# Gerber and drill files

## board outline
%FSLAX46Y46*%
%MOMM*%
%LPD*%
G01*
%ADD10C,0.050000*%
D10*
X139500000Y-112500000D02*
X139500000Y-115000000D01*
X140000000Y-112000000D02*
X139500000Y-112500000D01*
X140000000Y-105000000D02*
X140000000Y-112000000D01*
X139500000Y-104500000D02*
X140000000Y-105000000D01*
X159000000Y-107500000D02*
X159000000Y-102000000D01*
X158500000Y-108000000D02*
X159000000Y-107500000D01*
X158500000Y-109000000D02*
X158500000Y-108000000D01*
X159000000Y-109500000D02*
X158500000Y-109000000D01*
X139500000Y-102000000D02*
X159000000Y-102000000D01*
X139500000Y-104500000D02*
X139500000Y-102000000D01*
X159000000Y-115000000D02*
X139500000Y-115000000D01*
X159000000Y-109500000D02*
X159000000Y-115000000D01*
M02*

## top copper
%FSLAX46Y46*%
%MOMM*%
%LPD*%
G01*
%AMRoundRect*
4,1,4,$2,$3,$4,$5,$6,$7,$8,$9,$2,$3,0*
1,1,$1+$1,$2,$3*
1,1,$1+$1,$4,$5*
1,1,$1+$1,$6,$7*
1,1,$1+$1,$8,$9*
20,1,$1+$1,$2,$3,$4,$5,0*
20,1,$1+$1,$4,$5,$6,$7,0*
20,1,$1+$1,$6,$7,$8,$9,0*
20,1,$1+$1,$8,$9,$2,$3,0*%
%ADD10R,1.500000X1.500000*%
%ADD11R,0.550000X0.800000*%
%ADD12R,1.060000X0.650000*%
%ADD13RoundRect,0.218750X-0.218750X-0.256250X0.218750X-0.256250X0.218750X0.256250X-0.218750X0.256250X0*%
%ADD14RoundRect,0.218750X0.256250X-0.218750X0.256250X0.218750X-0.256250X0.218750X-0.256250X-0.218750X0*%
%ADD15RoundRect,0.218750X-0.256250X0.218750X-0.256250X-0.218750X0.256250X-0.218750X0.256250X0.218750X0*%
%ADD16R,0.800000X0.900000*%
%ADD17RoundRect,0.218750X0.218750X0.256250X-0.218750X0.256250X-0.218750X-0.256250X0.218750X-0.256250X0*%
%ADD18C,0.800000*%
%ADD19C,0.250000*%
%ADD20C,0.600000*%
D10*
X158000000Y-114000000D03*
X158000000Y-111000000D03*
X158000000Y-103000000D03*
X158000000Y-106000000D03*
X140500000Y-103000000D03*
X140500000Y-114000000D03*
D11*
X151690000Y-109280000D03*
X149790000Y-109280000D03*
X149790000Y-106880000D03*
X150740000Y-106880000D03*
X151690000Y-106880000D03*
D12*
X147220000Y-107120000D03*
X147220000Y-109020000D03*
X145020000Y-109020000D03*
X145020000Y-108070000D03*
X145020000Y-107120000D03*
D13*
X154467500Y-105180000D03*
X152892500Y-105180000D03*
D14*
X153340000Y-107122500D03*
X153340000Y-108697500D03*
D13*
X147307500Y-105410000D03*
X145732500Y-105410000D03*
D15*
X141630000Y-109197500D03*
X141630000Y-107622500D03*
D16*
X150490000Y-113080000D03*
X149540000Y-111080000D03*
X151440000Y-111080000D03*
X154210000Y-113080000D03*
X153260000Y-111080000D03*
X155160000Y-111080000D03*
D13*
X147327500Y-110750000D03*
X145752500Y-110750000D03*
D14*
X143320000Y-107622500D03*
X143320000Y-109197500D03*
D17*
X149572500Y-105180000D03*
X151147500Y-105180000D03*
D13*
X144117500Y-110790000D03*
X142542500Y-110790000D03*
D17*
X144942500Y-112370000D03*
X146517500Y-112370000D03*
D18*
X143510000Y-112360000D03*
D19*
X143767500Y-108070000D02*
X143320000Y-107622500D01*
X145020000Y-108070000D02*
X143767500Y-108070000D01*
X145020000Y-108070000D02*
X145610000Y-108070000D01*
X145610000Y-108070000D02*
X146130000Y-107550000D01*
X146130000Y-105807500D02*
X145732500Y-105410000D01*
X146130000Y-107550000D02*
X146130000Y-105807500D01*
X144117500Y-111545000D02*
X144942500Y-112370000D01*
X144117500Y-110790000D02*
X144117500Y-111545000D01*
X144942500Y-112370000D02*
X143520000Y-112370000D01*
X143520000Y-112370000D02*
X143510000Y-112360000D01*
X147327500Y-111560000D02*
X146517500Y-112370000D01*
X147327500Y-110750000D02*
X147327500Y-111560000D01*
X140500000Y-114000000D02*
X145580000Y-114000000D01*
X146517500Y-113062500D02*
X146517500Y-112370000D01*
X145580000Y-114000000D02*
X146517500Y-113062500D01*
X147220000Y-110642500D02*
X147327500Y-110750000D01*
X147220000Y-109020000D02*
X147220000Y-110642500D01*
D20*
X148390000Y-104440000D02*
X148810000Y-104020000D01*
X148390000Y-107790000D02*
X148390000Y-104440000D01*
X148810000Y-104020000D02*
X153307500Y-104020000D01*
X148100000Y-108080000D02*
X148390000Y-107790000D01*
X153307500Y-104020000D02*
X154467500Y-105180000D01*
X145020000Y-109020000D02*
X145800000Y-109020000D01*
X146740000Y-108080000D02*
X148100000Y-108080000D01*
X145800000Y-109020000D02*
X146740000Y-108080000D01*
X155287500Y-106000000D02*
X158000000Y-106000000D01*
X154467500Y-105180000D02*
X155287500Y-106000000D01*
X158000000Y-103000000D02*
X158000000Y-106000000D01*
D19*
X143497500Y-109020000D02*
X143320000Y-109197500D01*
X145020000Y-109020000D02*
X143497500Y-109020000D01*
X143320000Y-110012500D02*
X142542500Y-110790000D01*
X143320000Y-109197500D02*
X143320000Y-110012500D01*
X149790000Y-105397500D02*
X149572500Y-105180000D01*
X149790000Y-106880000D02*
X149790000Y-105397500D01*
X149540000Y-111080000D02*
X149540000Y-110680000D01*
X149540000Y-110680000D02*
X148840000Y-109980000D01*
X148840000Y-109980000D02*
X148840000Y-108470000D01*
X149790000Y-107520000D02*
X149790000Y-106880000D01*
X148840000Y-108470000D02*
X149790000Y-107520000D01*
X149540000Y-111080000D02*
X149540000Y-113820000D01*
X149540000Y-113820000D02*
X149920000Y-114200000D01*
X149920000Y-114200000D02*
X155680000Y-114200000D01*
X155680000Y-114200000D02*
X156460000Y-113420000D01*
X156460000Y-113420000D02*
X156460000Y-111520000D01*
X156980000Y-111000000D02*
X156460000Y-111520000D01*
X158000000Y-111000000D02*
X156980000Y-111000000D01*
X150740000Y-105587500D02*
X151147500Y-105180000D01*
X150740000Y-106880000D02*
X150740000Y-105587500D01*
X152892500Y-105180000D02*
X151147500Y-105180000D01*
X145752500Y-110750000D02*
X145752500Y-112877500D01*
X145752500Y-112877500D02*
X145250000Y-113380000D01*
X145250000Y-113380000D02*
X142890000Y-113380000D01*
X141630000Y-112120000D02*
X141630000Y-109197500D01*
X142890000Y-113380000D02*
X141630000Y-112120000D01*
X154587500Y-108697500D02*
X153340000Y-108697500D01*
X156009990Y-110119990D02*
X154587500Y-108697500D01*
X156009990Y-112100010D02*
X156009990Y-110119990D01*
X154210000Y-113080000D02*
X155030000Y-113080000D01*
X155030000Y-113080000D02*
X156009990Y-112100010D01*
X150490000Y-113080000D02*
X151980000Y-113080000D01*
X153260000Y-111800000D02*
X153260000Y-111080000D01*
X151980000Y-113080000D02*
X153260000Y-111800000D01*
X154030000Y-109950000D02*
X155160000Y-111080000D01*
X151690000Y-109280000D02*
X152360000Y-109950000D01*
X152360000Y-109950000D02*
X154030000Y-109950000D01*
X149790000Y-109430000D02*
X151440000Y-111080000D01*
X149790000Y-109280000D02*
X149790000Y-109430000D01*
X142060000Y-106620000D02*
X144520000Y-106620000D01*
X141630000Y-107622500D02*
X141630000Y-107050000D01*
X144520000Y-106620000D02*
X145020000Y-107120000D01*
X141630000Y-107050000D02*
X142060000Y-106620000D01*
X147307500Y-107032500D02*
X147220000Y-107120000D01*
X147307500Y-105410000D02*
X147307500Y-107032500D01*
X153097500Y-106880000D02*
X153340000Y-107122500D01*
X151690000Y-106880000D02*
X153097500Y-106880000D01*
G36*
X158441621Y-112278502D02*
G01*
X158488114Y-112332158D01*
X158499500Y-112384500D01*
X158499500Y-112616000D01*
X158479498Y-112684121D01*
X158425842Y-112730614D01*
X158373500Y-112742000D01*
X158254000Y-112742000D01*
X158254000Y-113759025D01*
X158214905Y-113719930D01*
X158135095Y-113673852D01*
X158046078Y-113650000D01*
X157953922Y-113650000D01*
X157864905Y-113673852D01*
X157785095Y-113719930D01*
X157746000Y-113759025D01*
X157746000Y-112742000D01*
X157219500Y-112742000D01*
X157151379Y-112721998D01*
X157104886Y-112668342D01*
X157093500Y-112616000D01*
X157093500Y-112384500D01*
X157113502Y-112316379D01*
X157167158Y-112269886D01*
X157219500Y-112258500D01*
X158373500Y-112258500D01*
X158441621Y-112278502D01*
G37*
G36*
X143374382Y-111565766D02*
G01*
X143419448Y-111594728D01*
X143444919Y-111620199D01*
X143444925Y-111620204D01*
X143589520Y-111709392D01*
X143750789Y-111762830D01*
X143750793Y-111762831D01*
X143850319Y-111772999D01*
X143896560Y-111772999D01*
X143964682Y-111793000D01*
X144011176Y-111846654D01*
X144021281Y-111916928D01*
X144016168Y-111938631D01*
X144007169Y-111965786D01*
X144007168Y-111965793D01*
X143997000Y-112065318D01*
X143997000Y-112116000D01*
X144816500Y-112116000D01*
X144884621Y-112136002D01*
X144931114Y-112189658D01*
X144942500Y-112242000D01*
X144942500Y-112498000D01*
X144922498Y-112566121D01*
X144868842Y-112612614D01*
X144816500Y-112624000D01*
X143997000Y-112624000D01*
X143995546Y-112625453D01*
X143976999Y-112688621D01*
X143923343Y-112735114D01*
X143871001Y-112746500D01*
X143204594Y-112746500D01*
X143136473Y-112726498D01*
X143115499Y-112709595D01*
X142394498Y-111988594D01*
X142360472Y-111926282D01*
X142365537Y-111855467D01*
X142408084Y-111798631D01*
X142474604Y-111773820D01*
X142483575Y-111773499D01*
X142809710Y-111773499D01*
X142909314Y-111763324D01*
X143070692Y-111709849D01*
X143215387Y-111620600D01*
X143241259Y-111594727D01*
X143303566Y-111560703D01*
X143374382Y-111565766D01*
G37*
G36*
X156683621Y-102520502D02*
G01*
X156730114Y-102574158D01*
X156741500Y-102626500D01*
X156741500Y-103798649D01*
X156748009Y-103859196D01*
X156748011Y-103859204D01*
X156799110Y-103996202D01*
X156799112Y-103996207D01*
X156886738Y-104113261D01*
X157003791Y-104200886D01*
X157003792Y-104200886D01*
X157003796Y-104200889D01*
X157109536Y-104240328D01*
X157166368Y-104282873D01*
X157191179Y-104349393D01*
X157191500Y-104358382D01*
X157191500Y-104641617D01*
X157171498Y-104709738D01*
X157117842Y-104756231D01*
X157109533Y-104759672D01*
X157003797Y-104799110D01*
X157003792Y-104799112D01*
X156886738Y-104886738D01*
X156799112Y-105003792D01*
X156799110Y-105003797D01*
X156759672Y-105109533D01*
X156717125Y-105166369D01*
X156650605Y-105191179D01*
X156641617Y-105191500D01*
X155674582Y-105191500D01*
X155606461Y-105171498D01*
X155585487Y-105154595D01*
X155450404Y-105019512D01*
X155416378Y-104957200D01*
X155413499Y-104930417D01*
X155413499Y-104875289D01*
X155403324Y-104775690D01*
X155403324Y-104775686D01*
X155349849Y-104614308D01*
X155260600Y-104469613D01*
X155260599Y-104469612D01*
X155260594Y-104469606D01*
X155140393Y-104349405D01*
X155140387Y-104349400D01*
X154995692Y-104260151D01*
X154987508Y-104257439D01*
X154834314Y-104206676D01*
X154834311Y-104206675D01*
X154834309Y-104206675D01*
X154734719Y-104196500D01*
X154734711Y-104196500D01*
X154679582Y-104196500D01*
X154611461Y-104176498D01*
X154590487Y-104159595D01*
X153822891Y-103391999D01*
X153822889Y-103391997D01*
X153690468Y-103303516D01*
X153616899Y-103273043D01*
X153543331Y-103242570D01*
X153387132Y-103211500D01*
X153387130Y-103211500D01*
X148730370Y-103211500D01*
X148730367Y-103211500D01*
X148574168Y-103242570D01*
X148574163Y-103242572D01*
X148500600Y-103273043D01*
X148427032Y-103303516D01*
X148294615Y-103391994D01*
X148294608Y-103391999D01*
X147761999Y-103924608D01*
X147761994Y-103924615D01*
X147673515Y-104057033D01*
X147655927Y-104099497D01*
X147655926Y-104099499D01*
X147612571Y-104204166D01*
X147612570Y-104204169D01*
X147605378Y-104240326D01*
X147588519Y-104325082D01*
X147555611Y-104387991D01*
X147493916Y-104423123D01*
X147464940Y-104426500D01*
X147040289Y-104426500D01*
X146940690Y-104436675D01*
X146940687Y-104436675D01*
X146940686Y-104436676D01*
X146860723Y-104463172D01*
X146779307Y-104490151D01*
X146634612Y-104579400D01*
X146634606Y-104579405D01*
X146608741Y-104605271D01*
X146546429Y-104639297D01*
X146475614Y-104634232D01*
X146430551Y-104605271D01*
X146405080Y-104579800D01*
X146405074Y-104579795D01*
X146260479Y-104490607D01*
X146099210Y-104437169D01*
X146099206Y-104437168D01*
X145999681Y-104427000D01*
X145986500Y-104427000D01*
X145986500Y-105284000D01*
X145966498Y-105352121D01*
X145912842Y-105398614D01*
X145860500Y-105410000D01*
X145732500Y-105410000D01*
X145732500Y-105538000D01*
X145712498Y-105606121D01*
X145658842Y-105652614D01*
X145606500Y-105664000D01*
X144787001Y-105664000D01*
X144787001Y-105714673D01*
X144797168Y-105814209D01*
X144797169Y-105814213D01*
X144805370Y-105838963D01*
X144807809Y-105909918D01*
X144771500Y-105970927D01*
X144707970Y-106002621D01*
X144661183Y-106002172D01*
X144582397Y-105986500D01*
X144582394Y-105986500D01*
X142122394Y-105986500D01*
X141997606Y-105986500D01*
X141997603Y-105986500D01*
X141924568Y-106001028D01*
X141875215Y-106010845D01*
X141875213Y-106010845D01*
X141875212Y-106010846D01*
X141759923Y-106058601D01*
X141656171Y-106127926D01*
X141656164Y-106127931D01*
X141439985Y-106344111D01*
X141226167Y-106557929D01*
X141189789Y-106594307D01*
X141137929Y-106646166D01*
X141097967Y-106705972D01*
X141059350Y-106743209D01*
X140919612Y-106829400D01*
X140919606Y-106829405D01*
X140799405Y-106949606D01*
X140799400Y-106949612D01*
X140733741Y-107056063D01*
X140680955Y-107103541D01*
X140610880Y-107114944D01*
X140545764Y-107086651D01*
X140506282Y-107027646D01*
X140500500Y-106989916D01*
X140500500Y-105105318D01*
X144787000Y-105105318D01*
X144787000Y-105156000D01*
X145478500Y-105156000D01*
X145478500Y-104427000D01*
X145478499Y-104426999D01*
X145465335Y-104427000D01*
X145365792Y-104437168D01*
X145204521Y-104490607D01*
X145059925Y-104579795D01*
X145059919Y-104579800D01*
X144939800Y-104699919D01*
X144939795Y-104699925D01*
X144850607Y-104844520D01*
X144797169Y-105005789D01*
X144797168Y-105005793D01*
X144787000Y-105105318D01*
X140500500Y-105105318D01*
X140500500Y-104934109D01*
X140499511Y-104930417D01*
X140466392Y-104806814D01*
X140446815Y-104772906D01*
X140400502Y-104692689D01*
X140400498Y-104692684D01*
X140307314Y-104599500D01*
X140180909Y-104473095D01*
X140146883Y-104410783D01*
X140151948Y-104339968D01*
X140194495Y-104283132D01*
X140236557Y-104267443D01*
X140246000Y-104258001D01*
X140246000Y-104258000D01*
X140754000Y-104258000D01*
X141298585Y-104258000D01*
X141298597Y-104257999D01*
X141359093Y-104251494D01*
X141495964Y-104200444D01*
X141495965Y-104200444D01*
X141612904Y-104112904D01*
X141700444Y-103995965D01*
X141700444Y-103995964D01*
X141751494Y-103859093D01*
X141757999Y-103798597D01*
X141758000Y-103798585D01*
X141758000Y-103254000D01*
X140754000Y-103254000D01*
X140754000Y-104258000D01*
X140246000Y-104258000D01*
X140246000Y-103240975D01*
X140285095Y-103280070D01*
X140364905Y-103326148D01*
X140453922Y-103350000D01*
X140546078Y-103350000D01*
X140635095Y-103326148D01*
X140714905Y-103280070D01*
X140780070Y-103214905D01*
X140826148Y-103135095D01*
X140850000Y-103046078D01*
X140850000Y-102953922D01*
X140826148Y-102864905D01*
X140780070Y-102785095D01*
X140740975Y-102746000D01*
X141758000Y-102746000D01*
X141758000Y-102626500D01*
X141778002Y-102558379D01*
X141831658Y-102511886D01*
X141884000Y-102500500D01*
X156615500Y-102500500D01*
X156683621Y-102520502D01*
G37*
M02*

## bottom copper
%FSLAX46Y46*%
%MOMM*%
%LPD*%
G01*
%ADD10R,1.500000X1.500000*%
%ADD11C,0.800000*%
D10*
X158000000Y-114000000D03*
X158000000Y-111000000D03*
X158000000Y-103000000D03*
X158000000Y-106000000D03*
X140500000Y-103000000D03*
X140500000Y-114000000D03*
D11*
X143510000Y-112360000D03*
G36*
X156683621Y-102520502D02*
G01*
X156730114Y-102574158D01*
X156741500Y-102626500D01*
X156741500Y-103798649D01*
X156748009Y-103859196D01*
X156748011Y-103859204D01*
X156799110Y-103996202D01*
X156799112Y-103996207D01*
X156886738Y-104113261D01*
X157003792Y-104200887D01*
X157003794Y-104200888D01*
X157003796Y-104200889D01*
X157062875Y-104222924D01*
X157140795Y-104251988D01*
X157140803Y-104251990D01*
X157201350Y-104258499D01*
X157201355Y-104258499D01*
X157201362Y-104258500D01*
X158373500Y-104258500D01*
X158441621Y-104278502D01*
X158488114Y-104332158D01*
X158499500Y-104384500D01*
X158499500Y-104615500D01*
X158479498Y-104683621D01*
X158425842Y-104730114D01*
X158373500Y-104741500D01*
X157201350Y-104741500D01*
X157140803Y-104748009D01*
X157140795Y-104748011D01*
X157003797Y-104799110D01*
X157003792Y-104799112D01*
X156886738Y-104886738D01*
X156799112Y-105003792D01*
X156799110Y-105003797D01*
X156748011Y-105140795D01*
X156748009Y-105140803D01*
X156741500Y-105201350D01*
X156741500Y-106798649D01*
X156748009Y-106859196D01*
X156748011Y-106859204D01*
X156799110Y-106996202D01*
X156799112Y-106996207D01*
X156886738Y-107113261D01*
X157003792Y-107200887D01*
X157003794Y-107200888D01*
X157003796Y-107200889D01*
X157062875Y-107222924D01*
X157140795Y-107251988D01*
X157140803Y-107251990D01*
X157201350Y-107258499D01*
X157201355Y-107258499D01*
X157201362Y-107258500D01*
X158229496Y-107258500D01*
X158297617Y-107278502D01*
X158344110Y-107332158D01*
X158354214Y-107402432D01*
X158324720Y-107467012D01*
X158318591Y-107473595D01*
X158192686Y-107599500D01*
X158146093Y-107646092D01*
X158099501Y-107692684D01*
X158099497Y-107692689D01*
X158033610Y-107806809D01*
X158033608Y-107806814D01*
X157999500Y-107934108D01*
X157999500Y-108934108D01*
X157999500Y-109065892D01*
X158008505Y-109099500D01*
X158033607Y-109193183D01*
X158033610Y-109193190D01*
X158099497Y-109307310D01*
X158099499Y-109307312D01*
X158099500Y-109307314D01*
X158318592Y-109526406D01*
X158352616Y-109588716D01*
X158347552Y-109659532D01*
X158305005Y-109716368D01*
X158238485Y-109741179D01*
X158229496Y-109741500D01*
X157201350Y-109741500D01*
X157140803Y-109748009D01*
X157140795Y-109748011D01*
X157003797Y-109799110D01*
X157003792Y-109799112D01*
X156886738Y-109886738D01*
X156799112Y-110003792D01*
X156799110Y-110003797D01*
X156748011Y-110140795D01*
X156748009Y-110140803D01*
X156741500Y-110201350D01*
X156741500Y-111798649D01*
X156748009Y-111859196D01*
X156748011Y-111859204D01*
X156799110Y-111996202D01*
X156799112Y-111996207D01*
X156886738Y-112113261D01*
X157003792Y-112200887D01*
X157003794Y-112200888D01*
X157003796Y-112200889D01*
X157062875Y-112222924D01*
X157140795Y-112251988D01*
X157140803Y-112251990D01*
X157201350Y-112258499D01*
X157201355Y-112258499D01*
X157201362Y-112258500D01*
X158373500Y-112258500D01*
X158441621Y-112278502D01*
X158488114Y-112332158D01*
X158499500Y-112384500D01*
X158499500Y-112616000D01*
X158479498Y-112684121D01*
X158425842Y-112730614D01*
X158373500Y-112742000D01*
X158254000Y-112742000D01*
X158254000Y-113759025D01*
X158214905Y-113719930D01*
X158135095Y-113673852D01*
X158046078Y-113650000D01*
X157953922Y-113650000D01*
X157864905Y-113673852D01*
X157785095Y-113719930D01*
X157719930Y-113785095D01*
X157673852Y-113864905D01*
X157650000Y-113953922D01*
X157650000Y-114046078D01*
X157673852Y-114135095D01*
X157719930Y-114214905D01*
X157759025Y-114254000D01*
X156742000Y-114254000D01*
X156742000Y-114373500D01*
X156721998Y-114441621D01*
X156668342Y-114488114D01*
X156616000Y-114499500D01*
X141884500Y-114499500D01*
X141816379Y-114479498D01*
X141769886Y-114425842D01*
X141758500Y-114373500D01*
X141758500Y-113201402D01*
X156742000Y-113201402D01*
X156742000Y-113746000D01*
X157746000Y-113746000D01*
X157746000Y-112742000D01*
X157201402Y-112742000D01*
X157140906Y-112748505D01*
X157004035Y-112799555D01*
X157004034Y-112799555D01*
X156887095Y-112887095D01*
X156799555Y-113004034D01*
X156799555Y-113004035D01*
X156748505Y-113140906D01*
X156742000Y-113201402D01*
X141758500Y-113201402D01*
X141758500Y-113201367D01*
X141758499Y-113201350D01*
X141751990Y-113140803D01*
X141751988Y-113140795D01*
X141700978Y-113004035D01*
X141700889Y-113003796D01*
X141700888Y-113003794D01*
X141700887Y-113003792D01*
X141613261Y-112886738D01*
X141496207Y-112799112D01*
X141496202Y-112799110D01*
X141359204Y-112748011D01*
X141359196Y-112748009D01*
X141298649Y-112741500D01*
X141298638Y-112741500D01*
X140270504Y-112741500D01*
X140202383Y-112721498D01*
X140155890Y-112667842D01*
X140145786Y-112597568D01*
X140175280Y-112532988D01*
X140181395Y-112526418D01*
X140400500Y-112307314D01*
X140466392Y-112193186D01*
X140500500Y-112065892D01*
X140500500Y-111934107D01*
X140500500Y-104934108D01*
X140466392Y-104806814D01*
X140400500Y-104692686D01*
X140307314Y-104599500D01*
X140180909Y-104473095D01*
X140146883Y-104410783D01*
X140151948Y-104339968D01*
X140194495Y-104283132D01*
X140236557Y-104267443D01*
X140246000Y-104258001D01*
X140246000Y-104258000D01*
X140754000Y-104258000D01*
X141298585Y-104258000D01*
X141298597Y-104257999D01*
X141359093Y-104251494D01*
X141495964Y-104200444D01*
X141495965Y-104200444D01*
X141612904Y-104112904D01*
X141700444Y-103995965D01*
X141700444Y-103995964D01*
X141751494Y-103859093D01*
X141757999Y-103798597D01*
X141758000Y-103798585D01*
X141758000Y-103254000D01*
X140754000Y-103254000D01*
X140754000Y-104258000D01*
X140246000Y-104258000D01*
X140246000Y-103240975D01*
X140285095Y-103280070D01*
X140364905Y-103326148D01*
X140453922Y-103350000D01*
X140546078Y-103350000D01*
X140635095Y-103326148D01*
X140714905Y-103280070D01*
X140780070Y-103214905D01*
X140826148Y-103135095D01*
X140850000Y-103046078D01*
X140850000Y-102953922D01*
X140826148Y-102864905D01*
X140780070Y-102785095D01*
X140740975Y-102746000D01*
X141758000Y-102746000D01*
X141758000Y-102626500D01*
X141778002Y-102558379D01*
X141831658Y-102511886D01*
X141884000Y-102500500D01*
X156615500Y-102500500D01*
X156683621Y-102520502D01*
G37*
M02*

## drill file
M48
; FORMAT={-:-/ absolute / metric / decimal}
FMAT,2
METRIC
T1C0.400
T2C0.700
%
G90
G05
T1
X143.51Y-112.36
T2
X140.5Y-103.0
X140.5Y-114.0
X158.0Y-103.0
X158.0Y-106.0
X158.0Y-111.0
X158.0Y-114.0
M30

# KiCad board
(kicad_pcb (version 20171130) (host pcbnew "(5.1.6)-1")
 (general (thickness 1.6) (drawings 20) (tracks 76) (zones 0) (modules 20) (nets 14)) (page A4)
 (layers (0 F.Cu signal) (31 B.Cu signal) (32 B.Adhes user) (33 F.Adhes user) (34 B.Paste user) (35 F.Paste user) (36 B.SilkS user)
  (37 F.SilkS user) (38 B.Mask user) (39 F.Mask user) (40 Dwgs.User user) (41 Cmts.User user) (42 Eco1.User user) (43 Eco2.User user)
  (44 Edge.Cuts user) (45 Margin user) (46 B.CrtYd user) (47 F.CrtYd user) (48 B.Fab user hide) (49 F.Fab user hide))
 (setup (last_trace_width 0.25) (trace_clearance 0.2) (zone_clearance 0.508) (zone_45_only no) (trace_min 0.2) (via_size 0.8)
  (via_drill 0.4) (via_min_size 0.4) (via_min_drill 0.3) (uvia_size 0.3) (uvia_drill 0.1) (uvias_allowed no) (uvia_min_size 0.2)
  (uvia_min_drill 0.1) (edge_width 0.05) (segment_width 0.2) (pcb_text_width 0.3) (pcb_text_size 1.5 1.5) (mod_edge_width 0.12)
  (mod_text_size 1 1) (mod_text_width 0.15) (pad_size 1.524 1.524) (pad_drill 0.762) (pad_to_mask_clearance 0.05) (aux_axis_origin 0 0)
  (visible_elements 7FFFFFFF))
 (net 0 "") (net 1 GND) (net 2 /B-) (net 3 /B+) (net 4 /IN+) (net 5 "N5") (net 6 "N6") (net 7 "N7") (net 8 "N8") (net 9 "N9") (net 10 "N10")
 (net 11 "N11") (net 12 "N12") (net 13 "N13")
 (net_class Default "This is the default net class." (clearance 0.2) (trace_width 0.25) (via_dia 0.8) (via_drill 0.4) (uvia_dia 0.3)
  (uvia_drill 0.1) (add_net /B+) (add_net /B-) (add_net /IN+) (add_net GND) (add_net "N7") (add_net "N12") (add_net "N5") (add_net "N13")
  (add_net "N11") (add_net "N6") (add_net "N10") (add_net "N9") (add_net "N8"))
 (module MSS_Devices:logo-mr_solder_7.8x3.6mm (layer B.Cu) (at 148.97 105.29 180)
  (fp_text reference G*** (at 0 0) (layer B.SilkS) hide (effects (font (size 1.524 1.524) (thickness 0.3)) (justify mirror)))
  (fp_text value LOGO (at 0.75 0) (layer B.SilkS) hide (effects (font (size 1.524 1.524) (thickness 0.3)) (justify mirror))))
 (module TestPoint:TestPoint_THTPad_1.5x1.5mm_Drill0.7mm (layer F.Cu) (at 158 114)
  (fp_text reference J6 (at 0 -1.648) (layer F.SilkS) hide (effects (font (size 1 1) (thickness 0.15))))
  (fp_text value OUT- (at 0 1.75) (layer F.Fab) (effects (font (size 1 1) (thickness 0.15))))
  (pad 1 thru_hole rect (at 0 0) (size 1.5 1.5) (drill 0.7) (layers *.Cu *.Mask) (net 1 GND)))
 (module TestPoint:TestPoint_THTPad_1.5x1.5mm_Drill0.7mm (layer F.Cu) (at 158 111)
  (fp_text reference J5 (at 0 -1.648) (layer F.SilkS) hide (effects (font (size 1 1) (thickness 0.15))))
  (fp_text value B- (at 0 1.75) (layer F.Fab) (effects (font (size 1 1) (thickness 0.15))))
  (pad 1 thru_hole rect (at 0 0) (size 1.5 1.5) (drill 0.7) (layers *.Cu *.Mask) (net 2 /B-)))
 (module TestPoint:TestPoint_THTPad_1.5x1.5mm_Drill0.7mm (layer F.Cu) (at 158 103)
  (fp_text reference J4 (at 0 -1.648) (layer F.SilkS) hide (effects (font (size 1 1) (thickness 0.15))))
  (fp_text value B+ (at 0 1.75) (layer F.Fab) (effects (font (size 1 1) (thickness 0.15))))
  (pad 1 thru_hole rect (at 0 0) (size 1.5 1.5) (drill 0.7) (layers *.Cu *.Mask) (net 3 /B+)))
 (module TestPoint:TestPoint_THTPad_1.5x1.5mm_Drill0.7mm (layer F.Cu) (at 158 106)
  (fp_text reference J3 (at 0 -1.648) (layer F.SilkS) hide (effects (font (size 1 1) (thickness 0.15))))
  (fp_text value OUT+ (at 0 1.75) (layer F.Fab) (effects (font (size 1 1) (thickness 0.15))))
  (pad 1 thru_hole rect (at 0 0) (size 1.5 1.5) (drill 0.7) (layers *.Cu *.Mask) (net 3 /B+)))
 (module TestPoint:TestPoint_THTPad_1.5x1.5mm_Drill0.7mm (layer F.Cu) (at 140.5 103)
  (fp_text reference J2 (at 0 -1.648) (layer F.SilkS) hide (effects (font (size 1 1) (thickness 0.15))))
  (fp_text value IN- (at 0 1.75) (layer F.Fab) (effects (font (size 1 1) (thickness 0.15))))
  (pad 1 thru_hole rect (at 0 0) (size 1.5 1.5) (drill 0.7) (layers *.Cu *.Mask) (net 1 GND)))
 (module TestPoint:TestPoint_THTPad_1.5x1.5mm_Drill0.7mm (layer F.Cu) (at 140.5 114)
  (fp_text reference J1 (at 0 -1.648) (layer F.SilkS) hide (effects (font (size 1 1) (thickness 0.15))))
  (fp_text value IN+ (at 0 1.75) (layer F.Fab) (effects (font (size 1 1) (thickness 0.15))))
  (pad 1 thru_hole rect (at 0 0) (size 1.5 1.5) (drill 0.7) (layers *.Cu *.Mask) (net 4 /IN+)))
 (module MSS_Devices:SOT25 (layer F.Cu) (at 150.74 108.08 180)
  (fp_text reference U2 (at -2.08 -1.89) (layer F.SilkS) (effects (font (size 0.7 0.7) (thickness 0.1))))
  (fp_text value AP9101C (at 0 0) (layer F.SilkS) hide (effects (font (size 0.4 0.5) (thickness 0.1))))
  (pad 5 smd rect (at -0.95 -1.2 180) (size 0.55 0.8) (layers F.Cu F.Paste F.Mask) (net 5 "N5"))
  (pad 4 smd rect (at 0.95 -1.2 180) (size 0.55 0.8) (layers F.Cu F.Paste F.Mask) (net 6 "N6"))
  (pad 3 smd rect (at 0.95 1.2 180) (size 0.55 0.8) (layers F.Cu F.Paste F.Mask) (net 2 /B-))
  (pad 2 smd rect (at 0 1.2 180) (size 0.55 0.8) (layers F.Cu F.Paste F.Mask) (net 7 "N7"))
  (pad 1 smd rect (at -0.95 1.2 180) (size 0.55 0.8) (layers F.Cu F.Paste F.Mask) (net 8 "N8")))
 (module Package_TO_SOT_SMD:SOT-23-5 (layer F.Cu) (at 146.12 108.07)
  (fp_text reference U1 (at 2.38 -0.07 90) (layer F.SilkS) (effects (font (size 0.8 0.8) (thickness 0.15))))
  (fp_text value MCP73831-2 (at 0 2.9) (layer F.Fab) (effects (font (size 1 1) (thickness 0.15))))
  (pad 5 smd rect (at 1.1 -0.95) (size 1.06 0.65) (layers F.Cu F.Paste F.Mask) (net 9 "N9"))
  (pad 4 smd rect (at 1.1 0.95) (size 1.06 0.65) (layers F.Cu F.Paste F.Mask) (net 4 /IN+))
  (pad 3 smd rect (at -1.1 0.95) (size 1.06 0.65) (layers F.Cu F.Paste F.Mask) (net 3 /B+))
  (pad 2 smd rect (at -1.1 0) (size 1.06 0.65) (layers F.Cu F.Paste F.Mask) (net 1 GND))
  (pad 1 smd rect (at -1.1 -0.95) (size 1.06 0.65) (layers F.Cu F.Paste F.Mask) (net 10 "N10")))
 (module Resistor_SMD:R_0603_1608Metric (layer F.Cu) (at 153.68 105.18)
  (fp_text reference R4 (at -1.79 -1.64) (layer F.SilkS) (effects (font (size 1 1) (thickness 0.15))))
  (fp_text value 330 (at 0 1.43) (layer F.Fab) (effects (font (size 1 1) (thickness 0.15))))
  (pad 2 smd roundrect (at 0.7875 0) (size 0.875 0.95) (layers F.Cu F.Paste F.Mask) (roundrect_rratio 0.25) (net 3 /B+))
  (pad 1 smd roundrect (at -0.7875 0) (size 0.875 0.95) (layers F.Cu F.Paste F.Mask) (roundrect_rratio 0.25) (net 7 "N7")))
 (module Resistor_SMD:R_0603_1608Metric (layer F.Cu) (at 153.34 107.91 90)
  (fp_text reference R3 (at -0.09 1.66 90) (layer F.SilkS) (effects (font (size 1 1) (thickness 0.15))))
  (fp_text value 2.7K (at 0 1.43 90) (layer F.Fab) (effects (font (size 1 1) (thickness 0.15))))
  (pad 2 smd roundrect (at 0.7875 0 90) (size 0.875 0.95) (layers F.Cu F.Paste F.Mask) (roundrect_rratio 0.25) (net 8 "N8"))
  (pad 1 smd roundrect (at -0.7875 0 90) (size 0.875 0.95) (layers F.Cu F.Paste F.Mask) (roundrect_rratio 0.25) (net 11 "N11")))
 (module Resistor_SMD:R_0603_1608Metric (layer F.Cu) (at 146.52 105.41)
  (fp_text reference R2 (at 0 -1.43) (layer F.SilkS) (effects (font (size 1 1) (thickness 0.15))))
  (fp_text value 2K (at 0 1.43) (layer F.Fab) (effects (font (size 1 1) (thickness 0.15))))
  (pad 2 smd roundrect (at 0.7875 0) (size 0.875 0.95) (layers F.Cu F.Paste F.Mask) (roundrect_rratio 0.25) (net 9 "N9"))
  (pad 1 smd roundrect (at -0.7875 0) (size 0.875 0.95) (layers F.Cu F.Paste F.Mask) (roundrect_rratio 0.25) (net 1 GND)))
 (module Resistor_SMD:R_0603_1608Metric (layer F.Cu) (at 141.63 108.41 270)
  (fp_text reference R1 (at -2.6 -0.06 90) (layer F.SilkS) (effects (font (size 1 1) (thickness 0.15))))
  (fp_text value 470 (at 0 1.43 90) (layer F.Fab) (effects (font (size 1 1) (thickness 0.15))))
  (pad 2 smd roundrect (at 0.7875 0 270) (size 0.875 0.95) (layers F.Cu F.Paste F.Mask) (roundrect_rratio 0.25) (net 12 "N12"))
  (pad 1 smd roundrect (at -0.7875 0 270) (size 0.875 0.95) (layers F.Cu F.Paste F.Mask) (roundrect_rratio 0.25) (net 10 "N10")))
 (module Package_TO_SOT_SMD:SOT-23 (layer F.Cu) (at 150.49 112.08 270)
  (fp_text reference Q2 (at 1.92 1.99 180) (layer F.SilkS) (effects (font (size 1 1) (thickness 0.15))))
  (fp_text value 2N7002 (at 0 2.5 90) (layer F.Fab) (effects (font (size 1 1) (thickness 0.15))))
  (pad 3 smd rect (at 1 0 270) (size 0.9 0.8) (layers F.Cu F.Paste F.Mask) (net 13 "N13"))
  (pad 2 smd rect (at -1 0.95 270) (size 0.9 0.8) (layers F.Cu F.Paste F.Mask) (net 2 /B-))
  (pad 1 smd rect (at -1 -0.95 270) (size 0.9 0.8) (layers F.Cu F.Paste F.Mask) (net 6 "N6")))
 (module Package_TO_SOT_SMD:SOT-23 (layer F.Cu) (at 154.21 112.08 270)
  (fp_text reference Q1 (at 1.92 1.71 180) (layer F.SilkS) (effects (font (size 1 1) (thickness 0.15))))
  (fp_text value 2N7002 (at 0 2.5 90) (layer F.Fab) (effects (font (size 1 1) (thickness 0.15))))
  (pad 3 smd rect (at 1 0 270) (size 0.9 0.8) (layers F.Cu F.Paste F.Mask) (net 11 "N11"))
  (pad 2 smd rect (at -1 0.95 270) (size 0.9 0.8) (layers F.Cu F.Paste F.Mask) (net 13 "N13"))
  (pad 1 smd rect (at -1 -0.95 270) (size 0.9 0.8) (layers F.Cu F.Paste F.Mask) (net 5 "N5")))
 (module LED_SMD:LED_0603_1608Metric (layer F.Cu) (at 146.54 110.75)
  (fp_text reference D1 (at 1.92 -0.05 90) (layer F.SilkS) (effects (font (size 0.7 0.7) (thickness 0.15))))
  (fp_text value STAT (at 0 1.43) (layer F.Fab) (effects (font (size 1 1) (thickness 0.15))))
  (pad 2 smd roundrect (at 0.7875 0) (size 0.875 0.95) (layers F.Cu F.Paste F.Mask) (roundrect_rratio 0.25) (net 4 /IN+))
  (pad 1 smd roundrect (at -0.7875 0) (size 0.875 0.95) (layers F.Cu F.Paste F.Mask) (roundrect_rratio 0.25) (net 12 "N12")))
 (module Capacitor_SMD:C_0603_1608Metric (layer F.Cu) (at 143.32 108.41 90)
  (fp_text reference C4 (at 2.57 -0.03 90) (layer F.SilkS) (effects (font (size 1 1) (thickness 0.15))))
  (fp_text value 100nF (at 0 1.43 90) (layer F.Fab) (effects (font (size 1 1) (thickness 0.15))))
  (pad 2 smd roundrect (at 0.7875 0 90) (size 0.875 0.95) (layers F.Cu F.Paste F.Mask) (roundrect_rratio 0.25) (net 1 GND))
  (pad 1 smd roundrect (at -0.7875 0 90) (size 0.875 0.95) (layers F.Cu F.Paste F.Mask) (roundrect_rratio 0.25) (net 3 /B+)))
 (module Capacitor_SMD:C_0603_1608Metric (layer F.Cu) (at 150.36 105.18 180)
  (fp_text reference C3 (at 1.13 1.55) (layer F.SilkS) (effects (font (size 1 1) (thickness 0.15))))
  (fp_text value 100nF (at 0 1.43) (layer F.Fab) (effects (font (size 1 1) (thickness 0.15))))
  (pad 2 smd roundrect (at 0.7875 0 180) (size 0.875 0.95) (layers F.Cu F.Paste F.Mask) (roundrect_rratio 0.25) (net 2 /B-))
  (pad 1 smd roundrect (at -0.7875 0 180) (size 0.875 0.95) (layers F.Cu F.Paste F.Mask) (roundrect_rratio 0.25) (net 7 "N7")))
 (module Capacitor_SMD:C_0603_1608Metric (layer F.Cu) (at 143.33 110.79)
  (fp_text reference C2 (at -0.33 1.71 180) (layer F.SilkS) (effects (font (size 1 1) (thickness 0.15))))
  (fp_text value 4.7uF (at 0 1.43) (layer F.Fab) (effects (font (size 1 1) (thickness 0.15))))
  (pad 2 smd roundrect (at 0.7875 0) (size 0.875 0.95) (layers F.Cu F.Paste F.Mask) (roundrect_rratio 0.25) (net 1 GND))
  (pad 1 smd roundrect (at -0.7875 0) (size 0.875 0.95) (layers F.Cu F.Paste F.Mask) (roundrect_rratio 0.25) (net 3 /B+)))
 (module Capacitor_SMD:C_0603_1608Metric (layer F.Cu) (at 145.73 112.37 180)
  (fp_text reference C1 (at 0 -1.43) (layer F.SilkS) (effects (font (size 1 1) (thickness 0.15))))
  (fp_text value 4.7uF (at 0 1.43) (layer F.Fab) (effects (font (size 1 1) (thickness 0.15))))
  (pad 2 smd roundrect (at 0.7875 0 180) (size 0.875 0.95) (layers F.Cu F.Paste F.Mask) (roundrect_rratio 0.25) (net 1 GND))
  (pad 1 smd roundrect (at -0.7875 0 180) (size 0.875 0.95) (layers F.Cu F.Paste F.Mask) (roundrect_rratio 0.25) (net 4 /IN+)))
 (gr_line (start 139.5 112.5) (end 139.5 115) (layer Edge.Cuts) (width 0.05))
 (gr_line (start 140 112) (end 139.5 112.5) (layer Edge.Cuts) (width 0.05))
 (gr_line (start 140 105) (end 140 112) (layer Edge.Cuts) (width 0.05))
 (gr_line (start 139.5 104.5) (end 140 105) (layer Edge.Cuts) (width 0.05))
 (gr_line (start 159 107.5) (end 159 102) (layer Edge.Cuts) (width 0.05))
 (gr_line (start 158.5 108) (end 159 107.5) (layer Edge.Cuts) (width 0.05))
 (gr_line (start 158.5 109) (end 158.5 108) (layer Edge.Cuts) (width 0.05))
 (gr_line (start 159 109.5) (end 158.5 109) (layer Edge.Cuts) (width 0.05))
 (gr_line (start 139.5 102) (end 159 102) (layer Edge.Cuts) (width 0.05))
 (gr_line (start 139.5 104.5) (end 139.5 102) (layer Edge.Cuts) (width 0.05))
 (gr_line (start 159 115) (end 139.5 115) (layer Edge.Cuts) (width 0.05))
 (gr_line (start 159 109.5) (end 159 115) (layer Edge.Cuts) (width 0.05))
 (segment (start 143.7675 108.07) (end 143.32 107.6225) (width 0.25) (layer F.Cu) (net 1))
 (segment (start 145.02 108.07) (end 143.7675 108.07) (width 0.25) (layer F.Cu) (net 1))
 (segment (start 145.02 108.07) (end 145.61 108.07) (width 0.25) (layer F.Cu) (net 1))
 (segment (start 145.61 108.07) (end 146.13 107.55) (width 0.25) (layer F.Cu) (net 1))
 (segment (start 146.13 105.8075) (end 145.7325 105.41) (width 0.25) (layer F.Cu) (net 1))
 (segment (start 146.13 107.55) (end 146.13 105.8075) (width 0.25) (layer F.Cu) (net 1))
 (segment (start 144.1175 111.545) (end 144.9425 112.37) (width 0.25) (layer F.Cu) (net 1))
 (segment (start 144.1175 110.79) (end 144.1175 111.545) (width 0.25) (layer F.Cu) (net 1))
 (via (at 143.51 112.36) (size 0.8) (drill 0.4) (layers F.Cu B.Cu) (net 1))
 (segment (start 144.9425 112.37) (end 143.52 112.37) (width 0.25) (layer F.Cu) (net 1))
 (segment (start 143.52 112.37) (end 143.51 112.36) (width 0.25) (layer F.Cu) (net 1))
 (segment (start 147.3275 111.56) (end 146.5175 112.37) (width 0.25) (layer F.Cu) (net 4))
 (segment (start 147.3275 110.75) (end 147.3275 111.56) (width 0.25) (layer F.Cu) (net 4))
 (segment (start 140.5 114) (end 145.58 114) (width 0.25) (layer F.Cu) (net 4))
 (segment (start 146.5175 113.0625) (end 146.5175 112.37) (width 0.25) (layer F.Cu) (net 4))
 (segment (start 145.58 114) (end 146.5175 113.0625) (width 0.25) (layer F.Cu) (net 4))
 (segment (start 147.22 110.6425) (end 147.3275 110.75) (width 0.25) (layer F.Cu) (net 4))
 (segment (start 147.22 109.02) (end 147.22 110.6425) (width 0.25) (layer F.Cu) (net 4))
 (segment (start 148.39 104.44) (end 148.81 104.02) (width 0.6) (layer F.Cu) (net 3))
 (segment (start 148.39 107.79) (end 148.39 104.44) (width 0.6) (layer F.Cu) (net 3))
 (segment (start 148.81 104.02) (end 153.3075 104.02) (width 0.6) (layer F.Cu) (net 3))
 (segment (start 148.1 108.08) (end 148.39 107.79) (width 0.6) (layer F.Cu) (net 3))
 (segment (start 153.3075 104.02) (end 154.4675 105.18) (width 0.6) (layer F.Cu) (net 3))
 (segment (start 145.02 109.02) (end 145.8 109.02) (width 0.6) (layer F.Cu) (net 3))
 (segment (start 146.74 108.08) (end 148.1 108.08) (width 0.6) (layer F.Cu) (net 3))
 (segment (start 145.8 109.02) (end 146.74 108.08) (width 0.6) (layer F.Cu) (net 3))
 (segment (start 155.2875 106) (end 158 106) (width 0.6) (layer F.Cu) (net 3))
 (segment (start 154.4675 105.18) (end 155.2875 106) (width 0.6) (layer F.Cu) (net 3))
 (segment (start 158 103) (end 158 106) (width 0.6) (layer F.Cu) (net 3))
 (segment (start 143.4975 109.02) (end 143.32 109.1975) (width 0.25) (layer F.Cu) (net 3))
 (segment (start 145.02 109.02) (end 143.4975 109.02) (width 0.25) (layer F.Cu) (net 3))
 (segment (start 143.32 110.0125) (end 142.5425 110.79) (width 0.25) (layer F.Cu) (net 3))
 (segment (start 143.32 109.1975) (end 143.32 110.0125) (width 0.25) (layer F.Cu) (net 3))
 (segment (start 149.79 105.3975) (end 149.5725 105.18) (width 0.25) (layer F.Cu) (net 2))
 (segment (start 149.79 106.88) (end 149.79 105.3975) (width 0.25) (layer F.Cu) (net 2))
 (segment (start 149.54 111.08) (end 149.54 110.68) (width 0.25) (layer F.Cu) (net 2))
 (segment (start 149.54 110.68) (end 148.84 109.98) (width 0.25) (layer F.Cu) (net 2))
 (segment (start 148.84 109.98) (end 148.84 108.47) (width 0.25) (layer F.Cu) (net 2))
 (segment (start 149.79 107.52) (end 149.79 106.88) (width 0.25) (layer F.Cu) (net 2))
 (segment (start 148.84 108.47) (end 149.79 107.52) (width 0.25) (layer F.Cu) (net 2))
 (segment (start 149.54 111.08) (end 149.54 113.82) (width 0.25) (layer F.Cu) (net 2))
 (segment (start 149.54 113.82) (end 149.92 114.2) (width 0.25) (layer F.Cu) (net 2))
 (segment (start 149.92 114.2) (end 155.68 114.2) (width 0.25) (layer F.Cu) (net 2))
 (segment (start 155.68 114.2) (end 156.46 113.42) (width 0.25) (layer F.Cu) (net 2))
 (segment (start 156.46 113.42) (end 156.46 111.52) (width 0.25) (layer F.Cu) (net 2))
 (segment (start 156.98 111) (end 156.46 111.52) (width 0.25) (layer F.Cu) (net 2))
 (segment (start 158 111) (end 156.98 111) (width 0.25) (layer F.Cu) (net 2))
 (segment (start 150.74 105.5875) (end 151.1475 105.18) (width 0.25) (layer F.Cu) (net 7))
 (segment (start 150.74 106.88) (end 150.74 105.5875) (width 0.25) (layer F.Cu) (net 7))
 (segment (start 152.8925 105.18) (end 151.1475 105.18) (width 0.25) (layer F.Cu) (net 7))
 (segment (start 145.7525 110.75) (end 145.7525 112.8775) (width 0.25) (layer F.Cu) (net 12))
 (segment (start 145.7525 112.8775) (end 145.25 113.38) (width 0.25) (layer F.Cu) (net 12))
 (segment (start 145.25 113.38) (end 142.89 113.38) (width 0.25) (layer F.Cu) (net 12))
 (segment (start 141.63 112.12) (end 141.63 109.1975) (width 0.25) (layer F.Cu) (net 12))
 (segment (start 142.89 113.38) (end 141.63 112.12) (width 0.25) (layer F.Cu) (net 12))
 (segment (start 154.5875 108.6975) (end 153.34 108.6975) (width 0.25) (layer F.Cu) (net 11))
 (segment (start 156.00999 110.11999) (end 154.5875 108.6975) (width 0.25) (layer F.Cu) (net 11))
 (segment (start 156.00999 112.10001) (end 156.00999 110.11999) (width 0.25) (layer F.Cu) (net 11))
 (segment (start 154.21 113.08) (end 155.03 113.08) (width 0.25) (layer F.Cu) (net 11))
 (segment (start 155.03 113.08) (end 156.00999 112.10001) (width 0.25) (layer F.Cu) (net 11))
 (segment (start 150.49 113.08) (end 151.98 113.08) (width 0.25) (layer F.Cu) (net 13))
 (segment (start 153.26 111.8) (end 153.26 111.08) (width 0.25) (layer F.Cu) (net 13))
 (segment (start 151.98 113.08) (end 153.26 111.8) (width 0.25) (layer F.Cu) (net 13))
 (segment (start 154.03 109.95) (end 155.16 111.08) (width 0.25) (layer F.Cu) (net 5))
 (segment (start 151.69 109.28) (end 152.36 109.95) (width 0.25) (layer F.Cu) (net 5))
 (segment (start 152.36 109.95) (end 154.03 109.95) (width 0.25) (layer F.Cu) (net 5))
 (segment (start 149.79 109.43) (end 151.44 111.08) (width 0.25) (layer F.Cu) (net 6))
 (segment (start 149.79 109.28) (end 149.79 109.43) (width 0.25) (layer F.Cu) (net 6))
 (segment (start 142.06 106.62) (end 144.52 106.62) (width 0.25) (layer F.Cu) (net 10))
 (segment (start 141.63 107.6225) (end 141.63 107.05) (width 0.25) (layer F.Cu) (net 10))
 (segment (start 144.52 106.62) (end 145.02 107.12) (width 0.25) (layer F.Cu) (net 10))
 (segment (start 141.63 107.05) (end 142.06 106.62) (width 0.25) (layer F.Cu) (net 10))
 (segment (start 147.3075 107.0325) (end 147.22 107.12) (width 0.25) (layer F.Cu) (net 9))
 (segment (start 147.3075 105.41) (end 147.3075 107.0325) (width 0.25) (layer F.Cu) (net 9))
 (segment (start 153.0975 106.88) (end 153.34 107.1225) (width 0.25) (layer F.Cu) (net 8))
 (segment (start 151.69 106.88) (end 153.0975 106.88) (width 0.25) (layer F.Cu) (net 8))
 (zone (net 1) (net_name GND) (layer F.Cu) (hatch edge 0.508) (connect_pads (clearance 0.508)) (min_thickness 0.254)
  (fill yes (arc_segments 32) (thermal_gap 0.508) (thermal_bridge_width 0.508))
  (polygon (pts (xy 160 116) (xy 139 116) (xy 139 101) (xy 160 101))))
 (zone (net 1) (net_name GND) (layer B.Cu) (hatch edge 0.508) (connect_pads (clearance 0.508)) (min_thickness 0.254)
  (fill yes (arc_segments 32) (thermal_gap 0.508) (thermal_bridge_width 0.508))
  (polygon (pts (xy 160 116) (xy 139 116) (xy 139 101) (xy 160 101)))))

